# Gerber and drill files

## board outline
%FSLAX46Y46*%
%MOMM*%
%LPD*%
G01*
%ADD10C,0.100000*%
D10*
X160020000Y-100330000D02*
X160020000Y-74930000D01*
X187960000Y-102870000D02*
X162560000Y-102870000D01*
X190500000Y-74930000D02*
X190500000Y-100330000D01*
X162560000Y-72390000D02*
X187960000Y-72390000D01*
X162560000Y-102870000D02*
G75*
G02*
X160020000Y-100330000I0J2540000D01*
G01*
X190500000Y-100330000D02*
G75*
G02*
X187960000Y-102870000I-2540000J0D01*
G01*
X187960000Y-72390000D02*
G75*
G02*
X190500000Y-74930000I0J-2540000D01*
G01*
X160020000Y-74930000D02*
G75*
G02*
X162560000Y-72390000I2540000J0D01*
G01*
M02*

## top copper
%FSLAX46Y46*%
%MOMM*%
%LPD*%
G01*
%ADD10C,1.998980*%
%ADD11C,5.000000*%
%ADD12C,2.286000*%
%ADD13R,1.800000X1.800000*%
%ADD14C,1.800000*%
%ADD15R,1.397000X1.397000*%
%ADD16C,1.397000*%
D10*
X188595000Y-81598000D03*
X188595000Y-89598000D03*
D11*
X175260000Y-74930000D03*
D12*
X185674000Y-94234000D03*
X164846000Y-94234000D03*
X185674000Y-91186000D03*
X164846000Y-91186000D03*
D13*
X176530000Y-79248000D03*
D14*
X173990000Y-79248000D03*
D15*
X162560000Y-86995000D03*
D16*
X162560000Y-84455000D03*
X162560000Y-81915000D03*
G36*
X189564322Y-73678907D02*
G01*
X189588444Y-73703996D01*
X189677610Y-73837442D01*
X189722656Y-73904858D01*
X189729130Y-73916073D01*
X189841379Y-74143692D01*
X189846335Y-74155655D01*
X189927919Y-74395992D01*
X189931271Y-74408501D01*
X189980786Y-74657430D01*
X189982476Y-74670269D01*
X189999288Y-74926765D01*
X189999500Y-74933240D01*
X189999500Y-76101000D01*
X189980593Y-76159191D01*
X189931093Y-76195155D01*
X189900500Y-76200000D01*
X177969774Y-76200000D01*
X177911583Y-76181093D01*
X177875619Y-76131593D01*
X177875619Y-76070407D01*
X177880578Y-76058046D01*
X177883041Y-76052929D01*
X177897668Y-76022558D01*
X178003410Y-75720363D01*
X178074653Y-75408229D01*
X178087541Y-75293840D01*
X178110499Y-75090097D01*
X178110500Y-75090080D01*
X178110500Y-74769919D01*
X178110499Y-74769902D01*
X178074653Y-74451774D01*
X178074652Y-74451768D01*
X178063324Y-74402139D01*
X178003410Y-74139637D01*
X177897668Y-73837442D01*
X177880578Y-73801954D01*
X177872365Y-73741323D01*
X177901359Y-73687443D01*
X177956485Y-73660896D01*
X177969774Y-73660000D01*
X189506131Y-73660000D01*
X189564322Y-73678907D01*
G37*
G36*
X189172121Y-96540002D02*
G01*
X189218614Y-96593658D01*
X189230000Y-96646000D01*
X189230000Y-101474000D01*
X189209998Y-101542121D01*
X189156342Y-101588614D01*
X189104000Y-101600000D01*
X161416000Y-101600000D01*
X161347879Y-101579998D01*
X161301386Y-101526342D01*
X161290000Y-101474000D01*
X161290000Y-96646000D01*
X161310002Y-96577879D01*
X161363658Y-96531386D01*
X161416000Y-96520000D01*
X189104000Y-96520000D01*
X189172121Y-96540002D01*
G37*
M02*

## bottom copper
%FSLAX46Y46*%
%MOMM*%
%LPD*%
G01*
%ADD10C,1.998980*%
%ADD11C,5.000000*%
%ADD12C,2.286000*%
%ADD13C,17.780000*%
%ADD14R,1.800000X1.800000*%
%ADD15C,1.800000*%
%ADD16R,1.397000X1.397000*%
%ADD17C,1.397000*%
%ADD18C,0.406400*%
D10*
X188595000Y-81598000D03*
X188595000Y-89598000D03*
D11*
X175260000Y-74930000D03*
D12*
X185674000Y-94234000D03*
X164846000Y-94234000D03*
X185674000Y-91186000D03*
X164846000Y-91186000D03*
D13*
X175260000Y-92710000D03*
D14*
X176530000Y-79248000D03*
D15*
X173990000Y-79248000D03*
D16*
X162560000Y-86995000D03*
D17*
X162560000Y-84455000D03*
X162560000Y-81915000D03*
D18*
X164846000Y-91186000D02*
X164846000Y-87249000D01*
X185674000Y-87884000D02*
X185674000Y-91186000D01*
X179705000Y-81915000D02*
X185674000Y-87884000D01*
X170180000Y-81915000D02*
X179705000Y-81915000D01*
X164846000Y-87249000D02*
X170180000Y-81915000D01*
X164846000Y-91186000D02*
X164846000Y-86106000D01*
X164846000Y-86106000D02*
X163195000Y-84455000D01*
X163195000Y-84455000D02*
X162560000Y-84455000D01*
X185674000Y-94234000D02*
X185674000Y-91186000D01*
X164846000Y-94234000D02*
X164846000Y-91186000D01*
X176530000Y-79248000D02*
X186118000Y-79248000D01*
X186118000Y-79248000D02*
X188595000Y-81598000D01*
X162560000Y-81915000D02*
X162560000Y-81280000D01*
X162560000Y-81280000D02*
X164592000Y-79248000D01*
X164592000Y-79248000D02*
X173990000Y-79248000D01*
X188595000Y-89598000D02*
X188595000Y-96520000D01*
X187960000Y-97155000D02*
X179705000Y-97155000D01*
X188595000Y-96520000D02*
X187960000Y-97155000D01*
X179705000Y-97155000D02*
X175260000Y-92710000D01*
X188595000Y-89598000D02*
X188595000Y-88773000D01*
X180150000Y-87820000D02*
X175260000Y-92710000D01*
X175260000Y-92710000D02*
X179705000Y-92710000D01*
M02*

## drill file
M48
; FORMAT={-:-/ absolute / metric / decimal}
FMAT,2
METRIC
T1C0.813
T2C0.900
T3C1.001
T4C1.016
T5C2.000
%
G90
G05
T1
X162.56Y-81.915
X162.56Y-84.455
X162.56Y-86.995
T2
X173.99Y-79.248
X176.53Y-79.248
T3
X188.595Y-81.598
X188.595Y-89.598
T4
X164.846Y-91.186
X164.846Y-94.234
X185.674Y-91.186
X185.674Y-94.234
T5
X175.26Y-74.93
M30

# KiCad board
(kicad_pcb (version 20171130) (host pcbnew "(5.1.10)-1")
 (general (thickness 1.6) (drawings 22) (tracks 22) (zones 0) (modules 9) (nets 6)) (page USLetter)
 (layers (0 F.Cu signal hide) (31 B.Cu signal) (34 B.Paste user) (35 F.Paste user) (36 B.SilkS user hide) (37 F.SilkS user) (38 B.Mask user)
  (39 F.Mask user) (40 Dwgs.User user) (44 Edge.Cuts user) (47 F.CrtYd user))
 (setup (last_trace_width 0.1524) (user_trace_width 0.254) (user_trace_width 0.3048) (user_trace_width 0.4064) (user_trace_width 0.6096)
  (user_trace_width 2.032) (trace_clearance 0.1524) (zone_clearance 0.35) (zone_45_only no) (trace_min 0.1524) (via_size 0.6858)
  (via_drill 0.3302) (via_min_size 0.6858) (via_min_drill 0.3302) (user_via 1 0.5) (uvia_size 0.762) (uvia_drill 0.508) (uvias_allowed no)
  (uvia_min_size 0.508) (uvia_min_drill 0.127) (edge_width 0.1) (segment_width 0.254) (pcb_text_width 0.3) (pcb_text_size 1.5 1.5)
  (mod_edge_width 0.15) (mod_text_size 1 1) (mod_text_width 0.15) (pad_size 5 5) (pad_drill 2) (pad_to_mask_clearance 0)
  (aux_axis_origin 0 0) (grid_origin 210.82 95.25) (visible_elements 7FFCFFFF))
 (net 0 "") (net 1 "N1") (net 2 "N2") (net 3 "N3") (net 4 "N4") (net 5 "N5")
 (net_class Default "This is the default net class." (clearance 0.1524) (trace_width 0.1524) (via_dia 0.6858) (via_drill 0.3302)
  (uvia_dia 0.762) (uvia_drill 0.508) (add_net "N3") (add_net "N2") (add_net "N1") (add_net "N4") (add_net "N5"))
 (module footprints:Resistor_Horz (layer F.Cu) (at 188.595 85.598 270)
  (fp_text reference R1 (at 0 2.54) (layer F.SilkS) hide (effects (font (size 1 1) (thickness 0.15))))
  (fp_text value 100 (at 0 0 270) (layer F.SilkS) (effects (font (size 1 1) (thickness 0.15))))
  (pad 1 thru_hole circle (at -4 0 270) (size 1.99898 1.99898) (drill 1.00076) (layers *.Cu *.SilkS *.Mask) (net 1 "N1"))
  (pad 2 thru_hole circle (at 4 0 270) (size 1.99898 1.99898) (drill 1.00076) (layers *.Cu *.SilkS *.Mask) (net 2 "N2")))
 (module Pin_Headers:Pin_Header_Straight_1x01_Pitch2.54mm (layer F.Cu) (at 175.26 74.93)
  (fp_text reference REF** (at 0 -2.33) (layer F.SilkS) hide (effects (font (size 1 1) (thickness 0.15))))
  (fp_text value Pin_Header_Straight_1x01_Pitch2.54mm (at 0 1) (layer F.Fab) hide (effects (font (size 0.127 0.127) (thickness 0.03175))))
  (pad 1 thru_hole circle (at 0 0) (size 5 5) (drill 2) (layers *.Cu B.Mask)))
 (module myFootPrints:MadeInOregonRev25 (layer F.Cu) (at 167.64 76.454)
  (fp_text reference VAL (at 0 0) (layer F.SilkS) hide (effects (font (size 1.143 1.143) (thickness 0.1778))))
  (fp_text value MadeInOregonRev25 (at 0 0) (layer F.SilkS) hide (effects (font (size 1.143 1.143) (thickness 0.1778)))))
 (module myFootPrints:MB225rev (layer F.Cu) (at 184.15 76.2)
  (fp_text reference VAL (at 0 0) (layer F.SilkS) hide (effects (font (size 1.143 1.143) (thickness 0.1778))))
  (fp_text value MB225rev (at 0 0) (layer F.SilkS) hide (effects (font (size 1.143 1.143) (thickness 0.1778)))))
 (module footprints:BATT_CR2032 (layer B.Cu) (at 175.26 92.71 180)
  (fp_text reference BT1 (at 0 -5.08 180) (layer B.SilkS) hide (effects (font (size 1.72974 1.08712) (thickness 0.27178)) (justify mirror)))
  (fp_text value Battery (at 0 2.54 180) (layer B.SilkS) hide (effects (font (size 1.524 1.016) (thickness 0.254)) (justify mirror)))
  (pad 1 thru_hole circle (at -10.414 -1.524 180) (size 2.286 2.286) (drill 1.016) (layers *.Cu *.Mask B.SilkS) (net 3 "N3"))
  (pad 1 thru_hole circle (at 10.414 -1.524 180) (size 2.286 2.286) (drill 1.016) (layers *.Cu *.Mask B.SilkS) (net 3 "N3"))
  (pad 1 thru_hole circle (at -10.414 1.524 180) (size 2.286 2.286) (drill 1.016) (layers *.Cu *.Mask B.SilkS) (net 3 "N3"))
  (pad 1 thru_hole circle (at 10.414 1.524 180) (size 2.286 2.286) (drill 1.016) (layers *.Cu *.Mask B.SilkS) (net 3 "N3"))
  (pad 2 smd circle (at 0 0 180) (size 17.78 17.78) (layers B.Cu B.Paste B.Mask) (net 2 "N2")))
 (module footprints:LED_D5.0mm (layer F.Cu) (at 176.53 79.248 180)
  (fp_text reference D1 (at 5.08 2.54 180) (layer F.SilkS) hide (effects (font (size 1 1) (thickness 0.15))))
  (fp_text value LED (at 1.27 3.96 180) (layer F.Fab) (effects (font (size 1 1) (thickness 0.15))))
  (pad 1 thru_hole rect (at 0 0 180) (size 1.8 1.8) (drill 0.9) (layers *.Cu *.Mask) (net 1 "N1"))
  (pad 2 thru_hole circle (at 2.54 0 180) (size 1.8 1.8) (drill 0.9) (layers *.Cu *.Mask) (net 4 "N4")))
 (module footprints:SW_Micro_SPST (layer F.Cu) (at 162.56 84.455 90)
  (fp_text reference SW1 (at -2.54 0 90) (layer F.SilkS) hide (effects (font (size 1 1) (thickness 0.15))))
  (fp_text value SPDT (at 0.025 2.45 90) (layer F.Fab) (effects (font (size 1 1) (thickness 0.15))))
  (pad 1 thru_hole rect (at -2.54 0 90) (size 1.397 1.397) (drill 0.8128) (layers *.Cu *.Mask F.SilkS) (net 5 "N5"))
  (pad 2 thru_hole circle (at 0 0 90) (size 1.397 1.397) (drill 0.8128) (layers *.Cu *.Mask F.SilkS) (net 3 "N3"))
  (pad 3 thru_hole circle (at 2.54 0 90) (size 1.397 1.397) (drill 0.8128) (layers *.Cu *.Mask F.SilkS) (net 4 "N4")))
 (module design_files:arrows (layer F.Cu) (at 179.07 77.47)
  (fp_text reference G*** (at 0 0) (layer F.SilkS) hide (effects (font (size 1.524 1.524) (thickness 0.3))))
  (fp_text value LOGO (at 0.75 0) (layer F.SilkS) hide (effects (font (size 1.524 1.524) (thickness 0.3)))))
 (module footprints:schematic (layer F.Cu) (at 175.26 87.503)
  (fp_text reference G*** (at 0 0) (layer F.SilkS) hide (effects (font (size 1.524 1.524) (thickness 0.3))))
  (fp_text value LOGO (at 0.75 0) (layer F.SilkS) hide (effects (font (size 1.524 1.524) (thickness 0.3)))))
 (gr_line (start 160.02 100.33) (end 160.02 74.93) (angle 90) (layer Edge.Cuts) (width 0.1))
 (gr_line (start 187.96 102.87) (end 162.56 102.87) (angle 90) (layer Edge.Cuts) (width 0.1))
 (gr_line (start 190.5 74.93) (end 190.5 100.33) (angle 90) (layer Edge.Cuts) (width 0.1))
 (gr_line (start 162.56 72.39) (end 187.96 72.39) (angle 90) (layer Edge.Cuts) (width 0.1))
 (gr_arc (start 162.56 100.33) (end 162.56 102.87) (angle 90) (layer Edge.Cuts) (width 0.1))
 (gr_arc (start 187.96 100.33) (end 190.5 100.33) (angle 90) (layer Edge.Cuts) (width 0.1))
 (gr_arc (start 187.96 74.93) (end 187.96 72.39) (angle 90) (layer Edge.Cuts) (width 0.1))
 (gr_arc (start 162.56 74.93) (end 160.02 74.93) (angle 90) (layer Edge.Cuts) (width 0.1))
 (segment (start 164.846 91.186) (end 164.846 87.249) (width 0.4064) (layer B.Cu) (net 3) (status 10))
 (segment (start 185.674 87.884) (end 185.674 91.186) (width 0.4064) (layer B.Cu) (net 3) (status 20))
 (segment (start 179.705 81.915) (end 185.674 87.884) (width 0.4064) (layer B.Cu) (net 3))
 (segment (start 170.18 81.915) (end 179.705 81.915) (width 0.4064) (layer B.Cu) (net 3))
 (segment (start 164.846 87.249) (end 170.18 81.915) (width 0.4064) (layer B.Cu) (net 3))
 (segment (start 164.846 91.186) (end 164.846 86.106) (width 0.4064) (layer B.Cu) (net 3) (status 10))
 (segment (start 164.846 86.106) (end 163.195 84.455) (width 0.4064) (layer B.Cu) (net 3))
 (segment (start 163.195 84.455) (end 162.56 84.455) (width 0.4064) (layer B.Cu) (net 3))
 (segment (start 185.674 94.234) (end 185.674 91.186) (width 0.4064) (layer B.Cu) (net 3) (status 30))
 (segment (start 164.846 94.234) (end 164.846 91.186) (width 0.4064) (layer B.Cu) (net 3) (status 30))
 (segment (start 176.53 79.248) (end 186.118 79.248) (width 0.4064) (layer B.Cu) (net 1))
 (segment (start 186.118 79.248) (end 188.595 81.598) (width 0.4064) (layer B.Cu) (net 1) (status 20))
 (segment (start 162.56 81.915) (end 162.56 81.28) (width 0.4064) (layer B.Cu) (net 4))
 (segment (start 162.56 81.28) (end 164.592 79.248) (width 0.4064) (layer B.Cu) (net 4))
 (segment (start 164.592 79.248) (end 173.99 79.248) (width 0.4064) (layer B.Cu) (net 4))
 (segment (start 188.595 89.598) (end 188.595 96.52) (width 0.4064) (layer B.Cu) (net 2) (status 10))
 (segment (start 187.96 97.155) (end 179.705 97.155) (width 0.4064) (layer B.Cu) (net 2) (status 20))
 (segment (start 188.595 96.52) (end 187.96 97.155) (width 0.4064) (layer B.Cu) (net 2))
 (segment (start 179.705 97.155) (end 175.26 92.71) (width 0.4064) (layer B.Cu) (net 2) (status 30))
 (segment (start 188.595 89.598) (end 188.595 88.773) (width 0.4064) (layer B.Cu) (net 2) (status 30))
 (segment (start 180.15 87.82) (end 175.26 92.71) (width 0.4064) (layer B.Cu) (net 2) (status 30))
 (segment (start 175.26 92.71) (end 179.705 92.71) (width 0.4064) (layer B.Cu) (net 2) (status 30))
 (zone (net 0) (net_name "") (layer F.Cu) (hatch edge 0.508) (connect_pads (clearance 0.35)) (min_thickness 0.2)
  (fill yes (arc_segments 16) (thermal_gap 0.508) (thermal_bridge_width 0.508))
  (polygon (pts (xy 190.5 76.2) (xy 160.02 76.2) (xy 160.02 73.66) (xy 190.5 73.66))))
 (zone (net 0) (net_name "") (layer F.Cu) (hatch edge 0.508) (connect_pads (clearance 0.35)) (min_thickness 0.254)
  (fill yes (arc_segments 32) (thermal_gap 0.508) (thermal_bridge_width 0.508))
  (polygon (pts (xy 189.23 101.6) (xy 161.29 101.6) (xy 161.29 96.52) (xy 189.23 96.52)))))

